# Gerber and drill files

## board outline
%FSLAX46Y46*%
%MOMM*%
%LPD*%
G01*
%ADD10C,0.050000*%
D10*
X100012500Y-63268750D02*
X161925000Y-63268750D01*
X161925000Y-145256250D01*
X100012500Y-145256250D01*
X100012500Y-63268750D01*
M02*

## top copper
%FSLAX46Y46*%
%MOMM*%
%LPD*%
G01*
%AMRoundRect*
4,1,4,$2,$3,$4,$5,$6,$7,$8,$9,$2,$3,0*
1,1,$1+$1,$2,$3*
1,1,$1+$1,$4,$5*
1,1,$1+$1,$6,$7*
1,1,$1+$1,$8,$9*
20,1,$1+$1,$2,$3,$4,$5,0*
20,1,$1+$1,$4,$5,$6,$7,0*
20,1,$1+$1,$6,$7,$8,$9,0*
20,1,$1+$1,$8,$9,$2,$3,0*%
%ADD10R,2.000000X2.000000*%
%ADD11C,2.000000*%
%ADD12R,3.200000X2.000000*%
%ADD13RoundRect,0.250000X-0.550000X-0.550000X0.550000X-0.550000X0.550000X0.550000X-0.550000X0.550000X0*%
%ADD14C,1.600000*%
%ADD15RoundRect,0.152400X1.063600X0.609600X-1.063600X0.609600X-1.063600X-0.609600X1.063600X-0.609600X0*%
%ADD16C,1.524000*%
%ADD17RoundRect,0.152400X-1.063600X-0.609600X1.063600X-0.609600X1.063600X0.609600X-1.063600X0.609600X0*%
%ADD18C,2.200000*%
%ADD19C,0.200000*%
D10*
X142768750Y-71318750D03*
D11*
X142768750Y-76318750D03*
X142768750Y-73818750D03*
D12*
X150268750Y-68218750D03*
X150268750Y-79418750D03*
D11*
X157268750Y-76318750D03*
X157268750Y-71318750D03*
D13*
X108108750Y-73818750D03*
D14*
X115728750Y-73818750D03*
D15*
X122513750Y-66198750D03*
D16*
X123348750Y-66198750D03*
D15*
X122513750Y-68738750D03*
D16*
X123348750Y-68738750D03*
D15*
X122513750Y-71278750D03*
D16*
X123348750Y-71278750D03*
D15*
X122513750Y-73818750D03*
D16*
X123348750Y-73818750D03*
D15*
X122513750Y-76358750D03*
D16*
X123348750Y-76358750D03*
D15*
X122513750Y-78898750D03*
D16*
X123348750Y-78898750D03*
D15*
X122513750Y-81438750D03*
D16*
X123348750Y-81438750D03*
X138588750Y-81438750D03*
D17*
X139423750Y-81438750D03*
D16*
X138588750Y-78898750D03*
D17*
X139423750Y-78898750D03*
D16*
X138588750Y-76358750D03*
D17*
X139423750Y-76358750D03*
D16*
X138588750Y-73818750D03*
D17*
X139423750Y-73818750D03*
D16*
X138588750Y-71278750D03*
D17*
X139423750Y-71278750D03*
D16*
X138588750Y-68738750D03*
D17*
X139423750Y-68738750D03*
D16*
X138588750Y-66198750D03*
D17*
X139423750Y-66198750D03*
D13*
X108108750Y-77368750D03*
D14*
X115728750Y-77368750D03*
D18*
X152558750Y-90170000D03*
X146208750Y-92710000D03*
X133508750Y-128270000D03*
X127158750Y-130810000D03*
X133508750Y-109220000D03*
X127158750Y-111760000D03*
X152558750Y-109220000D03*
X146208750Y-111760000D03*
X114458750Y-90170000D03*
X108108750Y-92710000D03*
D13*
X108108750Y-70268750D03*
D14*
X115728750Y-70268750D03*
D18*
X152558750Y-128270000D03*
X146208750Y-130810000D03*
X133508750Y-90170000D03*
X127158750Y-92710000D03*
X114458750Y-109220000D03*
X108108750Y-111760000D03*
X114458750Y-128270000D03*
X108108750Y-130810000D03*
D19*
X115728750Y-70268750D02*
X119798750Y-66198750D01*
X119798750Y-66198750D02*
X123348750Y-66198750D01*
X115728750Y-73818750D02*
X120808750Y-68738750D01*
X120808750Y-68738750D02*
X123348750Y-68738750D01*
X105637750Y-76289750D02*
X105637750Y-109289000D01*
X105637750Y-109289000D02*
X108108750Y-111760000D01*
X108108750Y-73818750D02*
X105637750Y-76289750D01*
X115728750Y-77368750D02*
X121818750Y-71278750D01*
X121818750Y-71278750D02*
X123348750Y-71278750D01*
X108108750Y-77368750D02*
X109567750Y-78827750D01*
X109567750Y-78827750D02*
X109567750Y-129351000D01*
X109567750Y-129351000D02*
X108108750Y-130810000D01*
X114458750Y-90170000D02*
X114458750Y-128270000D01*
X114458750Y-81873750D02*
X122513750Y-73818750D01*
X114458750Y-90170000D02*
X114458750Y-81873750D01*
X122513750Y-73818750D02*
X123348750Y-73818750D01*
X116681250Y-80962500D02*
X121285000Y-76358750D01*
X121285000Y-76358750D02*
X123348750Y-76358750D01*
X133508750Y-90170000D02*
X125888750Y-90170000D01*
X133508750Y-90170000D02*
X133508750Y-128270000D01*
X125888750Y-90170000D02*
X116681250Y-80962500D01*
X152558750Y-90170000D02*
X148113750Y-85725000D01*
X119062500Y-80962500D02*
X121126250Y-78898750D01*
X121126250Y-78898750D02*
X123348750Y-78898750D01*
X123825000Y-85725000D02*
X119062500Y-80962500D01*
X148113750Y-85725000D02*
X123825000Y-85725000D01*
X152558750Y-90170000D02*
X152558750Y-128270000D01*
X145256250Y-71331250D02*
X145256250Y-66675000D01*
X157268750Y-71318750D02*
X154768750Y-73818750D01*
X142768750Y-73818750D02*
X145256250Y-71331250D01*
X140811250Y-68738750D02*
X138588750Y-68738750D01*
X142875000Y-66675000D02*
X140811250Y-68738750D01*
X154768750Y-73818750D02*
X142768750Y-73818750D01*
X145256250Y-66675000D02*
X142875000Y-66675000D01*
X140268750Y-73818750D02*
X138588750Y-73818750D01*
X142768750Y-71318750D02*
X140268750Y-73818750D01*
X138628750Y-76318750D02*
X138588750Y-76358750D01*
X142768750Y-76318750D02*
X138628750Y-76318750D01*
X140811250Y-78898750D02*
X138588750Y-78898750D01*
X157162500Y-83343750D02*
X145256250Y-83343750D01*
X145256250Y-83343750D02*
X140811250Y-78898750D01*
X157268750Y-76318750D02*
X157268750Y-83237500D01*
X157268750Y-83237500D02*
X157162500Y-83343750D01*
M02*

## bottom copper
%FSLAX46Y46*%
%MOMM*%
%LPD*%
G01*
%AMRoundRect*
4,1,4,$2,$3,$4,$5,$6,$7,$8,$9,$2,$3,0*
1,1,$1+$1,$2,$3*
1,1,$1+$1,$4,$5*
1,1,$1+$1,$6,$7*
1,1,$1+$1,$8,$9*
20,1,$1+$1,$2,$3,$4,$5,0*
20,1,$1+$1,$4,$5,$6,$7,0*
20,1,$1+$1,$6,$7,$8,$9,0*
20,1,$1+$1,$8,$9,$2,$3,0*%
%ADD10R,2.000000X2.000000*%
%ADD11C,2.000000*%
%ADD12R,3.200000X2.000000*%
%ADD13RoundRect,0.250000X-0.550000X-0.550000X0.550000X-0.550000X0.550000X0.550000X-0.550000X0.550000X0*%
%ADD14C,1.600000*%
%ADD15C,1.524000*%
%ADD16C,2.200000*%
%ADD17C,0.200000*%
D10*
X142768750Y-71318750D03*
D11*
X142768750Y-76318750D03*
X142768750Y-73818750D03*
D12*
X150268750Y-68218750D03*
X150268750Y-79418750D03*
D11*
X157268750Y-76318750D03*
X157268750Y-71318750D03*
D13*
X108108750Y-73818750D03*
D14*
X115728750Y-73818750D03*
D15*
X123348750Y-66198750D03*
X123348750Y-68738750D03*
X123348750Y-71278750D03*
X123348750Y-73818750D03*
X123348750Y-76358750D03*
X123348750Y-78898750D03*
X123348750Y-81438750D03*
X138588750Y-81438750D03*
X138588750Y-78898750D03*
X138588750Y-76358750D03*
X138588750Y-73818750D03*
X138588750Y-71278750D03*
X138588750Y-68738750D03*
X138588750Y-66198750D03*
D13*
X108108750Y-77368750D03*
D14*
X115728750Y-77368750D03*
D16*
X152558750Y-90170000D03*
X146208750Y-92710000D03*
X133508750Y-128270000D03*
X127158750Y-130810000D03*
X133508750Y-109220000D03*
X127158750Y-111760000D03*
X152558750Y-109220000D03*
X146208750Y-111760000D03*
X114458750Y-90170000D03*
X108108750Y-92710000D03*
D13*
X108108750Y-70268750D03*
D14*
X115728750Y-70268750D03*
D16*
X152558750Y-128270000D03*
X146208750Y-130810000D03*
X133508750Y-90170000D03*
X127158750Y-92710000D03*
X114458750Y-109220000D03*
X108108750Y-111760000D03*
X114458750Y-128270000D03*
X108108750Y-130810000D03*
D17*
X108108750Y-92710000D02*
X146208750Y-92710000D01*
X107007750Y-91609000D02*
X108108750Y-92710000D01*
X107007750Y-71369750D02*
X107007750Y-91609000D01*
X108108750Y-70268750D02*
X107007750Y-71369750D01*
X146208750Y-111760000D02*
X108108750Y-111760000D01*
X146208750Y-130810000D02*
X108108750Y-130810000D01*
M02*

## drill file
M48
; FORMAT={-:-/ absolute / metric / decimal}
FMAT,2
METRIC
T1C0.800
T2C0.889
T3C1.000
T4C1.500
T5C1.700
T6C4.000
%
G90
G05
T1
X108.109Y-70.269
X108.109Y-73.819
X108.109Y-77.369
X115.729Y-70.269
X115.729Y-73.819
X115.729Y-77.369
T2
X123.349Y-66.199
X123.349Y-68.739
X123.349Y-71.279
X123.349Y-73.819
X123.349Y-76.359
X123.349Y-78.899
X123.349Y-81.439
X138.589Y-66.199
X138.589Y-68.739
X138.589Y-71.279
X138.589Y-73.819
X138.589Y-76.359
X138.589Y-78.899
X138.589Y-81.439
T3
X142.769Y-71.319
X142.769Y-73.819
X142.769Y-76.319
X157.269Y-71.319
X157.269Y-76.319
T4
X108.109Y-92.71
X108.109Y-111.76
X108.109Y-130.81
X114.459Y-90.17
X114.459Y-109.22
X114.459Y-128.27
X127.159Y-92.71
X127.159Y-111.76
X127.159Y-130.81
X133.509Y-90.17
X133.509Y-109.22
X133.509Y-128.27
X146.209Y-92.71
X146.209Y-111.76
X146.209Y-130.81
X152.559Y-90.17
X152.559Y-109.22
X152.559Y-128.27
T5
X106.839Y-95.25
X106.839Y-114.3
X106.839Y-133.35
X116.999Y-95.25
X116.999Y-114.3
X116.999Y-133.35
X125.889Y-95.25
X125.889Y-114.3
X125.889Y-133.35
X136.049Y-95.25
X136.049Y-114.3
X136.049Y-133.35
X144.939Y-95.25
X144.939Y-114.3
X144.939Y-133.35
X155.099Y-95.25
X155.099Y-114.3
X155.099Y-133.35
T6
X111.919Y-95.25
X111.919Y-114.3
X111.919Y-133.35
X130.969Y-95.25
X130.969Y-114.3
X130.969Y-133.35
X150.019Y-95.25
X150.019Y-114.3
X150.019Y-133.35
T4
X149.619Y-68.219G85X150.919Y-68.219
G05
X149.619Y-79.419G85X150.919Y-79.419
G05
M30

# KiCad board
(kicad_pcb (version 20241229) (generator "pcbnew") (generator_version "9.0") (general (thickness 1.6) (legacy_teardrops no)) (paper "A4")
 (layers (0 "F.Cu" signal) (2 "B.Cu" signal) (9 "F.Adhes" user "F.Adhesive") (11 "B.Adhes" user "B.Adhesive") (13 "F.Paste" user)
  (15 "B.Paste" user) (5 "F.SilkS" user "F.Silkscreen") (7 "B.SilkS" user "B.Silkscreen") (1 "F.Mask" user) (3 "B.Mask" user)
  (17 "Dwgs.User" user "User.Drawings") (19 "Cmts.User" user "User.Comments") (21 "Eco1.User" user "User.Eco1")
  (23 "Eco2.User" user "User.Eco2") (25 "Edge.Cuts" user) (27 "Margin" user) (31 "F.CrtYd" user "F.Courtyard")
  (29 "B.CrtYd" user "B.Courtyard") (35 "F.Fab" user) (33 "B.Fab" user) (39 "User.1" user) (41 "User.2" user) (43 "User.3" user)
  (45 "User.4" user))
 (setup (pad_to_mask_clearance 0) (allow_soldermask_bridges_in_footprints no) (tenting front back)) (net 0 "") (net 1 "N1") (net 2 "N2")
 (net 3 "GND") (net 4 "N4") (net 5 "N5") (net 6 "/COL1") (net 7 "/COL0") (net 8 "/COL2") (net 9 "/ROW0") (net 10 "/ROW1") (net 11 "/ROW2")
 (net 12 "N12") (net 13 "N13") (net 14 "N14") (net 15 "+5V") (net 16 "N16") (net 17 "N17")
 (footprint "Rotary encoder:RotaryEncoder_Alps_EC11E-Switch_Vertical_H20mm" (layer "F.Cu") (at 142.76875 71.31875)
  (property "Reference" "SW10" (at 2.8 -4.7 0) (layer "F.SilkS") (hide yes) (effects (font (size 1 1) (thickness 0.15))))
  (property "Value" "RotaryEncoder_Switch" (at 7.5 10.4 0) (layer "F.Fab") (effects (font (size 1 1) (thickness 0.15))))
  (pad "A" thru_hole rect (at 0 0) (size 2 2) (drill 1) (layers "*.Cu" "*.Mask") (remove_unused_layers no) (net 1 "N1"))
  (pad "B" thru_hole circle (at 0 5) (size 2 2) (drill 1) (layers "*.Cu" "*.Mask") (remove_unused_layers no) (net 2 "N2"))
  (pad "C" thru_hole circle (at 0 2.5) (size 2 2) (drill 1) (layers "*.Cu" "*.Mask") (remove_unused_layers no) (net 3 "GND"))
  (pad "MP" thru_hole rect (at 7.5 -3.1) (size 3.2 2) (drill oval 2.8 1.5) (layers "*.Cu" "*.Mask") (remove_unused_layers no))
  (pad "MP" thru_hole rect (at 7.5 8.1) (size 3.2 2) (drill oval 2.8 1.5) (layers "*.Cu" "*.Mask") (remove_unused_layers no))
  (pad "S1" thru_hole circle (at 14.5 5) (size 2 2) (drill 1) (layers "*.Cu" "*.Mask") (remove_unused_layers no) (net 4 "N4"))
  (pad "S2" thru_hole circle (at 14.5 0) (size 2 2) (drill 1) (layers "*.Cu" "*.Mask") (remove_unused_layers no) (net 3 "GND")))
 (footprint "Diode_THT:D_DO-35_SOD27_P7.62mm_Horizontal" (layer "F.Cu") (at 108.10875 73.81875)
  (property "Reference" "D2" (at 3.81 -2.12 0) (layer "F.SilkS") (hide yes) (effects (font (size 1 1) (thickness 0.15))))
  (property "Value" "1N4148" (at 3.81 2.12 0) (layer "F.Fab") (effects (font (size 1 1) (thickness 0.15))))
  (pad "1" thru_hole roundrect (at 0 0) (size 1.6 1.6) (drill 0.8) (layers "*.Cu" "*.Mask") (remove_unused_layers no)
   (roundrect_rratio 0.15625) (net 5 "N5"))
  (pad "2" thru_hole circle (at 7.62 0) (size 1.6 1.6) (drill 0.8) (layers "*.Cu" "*.Mask") (remove_unused_layers no) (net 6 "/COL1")))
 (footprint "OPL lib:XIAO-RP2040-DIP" (layer "F.Cu") (at 130.96875 73.81875)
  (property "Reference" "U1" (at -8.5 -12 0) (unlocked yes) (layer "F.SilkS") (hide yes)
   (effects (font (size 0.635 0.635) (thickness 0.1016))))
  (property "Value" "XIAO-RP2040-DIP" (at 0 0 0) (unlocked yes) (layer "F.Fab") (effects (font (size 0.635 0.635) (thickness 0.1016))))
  (pad "1" smd roundrect (at -8.455 -7.62 180) (size 2.432 1.524) (layers "F.Cu" "F.Mask") (roundrect_rratio 0.1) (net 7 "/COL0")
   (thermal_bridge_angle 45))
  (pad "1" thru_hole circle (at -7.62 -7.62 180) (size 1.524 1.524) (drill 0.889) (layers "*.Cu" "*.Mask") (remove_unused_layers no)
   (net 7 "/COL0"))
  (pad "2" smd roundrect (at -8.455 -5.08 180) (size 2.432 1.524) (layers "F.Cu" "F.Mask") (roundrect_rratio 0.1) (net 6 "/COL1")
   (thermal_bridge_angle 45))
  (pad "2" thru_hole circle (at -7.62 -5.08 180) (size 1.524 1.524) (drill 0.889) (layers "*.Cu" "*.Mask") (remove_unused_layers no)
   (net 6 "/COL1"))
  (pad "3" smd roundrect (at -8.455 -2.54 180) (size 2.432 1.524) (layers "F.Cu" "F.Mask") (roundrect_rratio 0.1) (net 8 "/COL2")
   (thermal_bridge_angle 45))
  (pad "3" thru_hole circle (at -7.62 -2.54 180) (size 1.524 1.524) (drill 0.889) (layers "*.Cu" "*.Mask") (remove_unused_layers no)
   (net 8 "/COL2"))
  (pad "4" smd roundrect (at -8.455 0 180) (size 2.432 1.524) (layers "F.Cu" "F.Mask") (roundrect_rratio 0.1) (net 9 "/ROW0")
   (thermal_bridge_angle 45))
  (pad "4" thru_hole circle (at -7.62 0 180) (size 1.524 1.524) (drill 0.889) (layers "*.Cu" "*.Mask") (remove_unused_layers no)
   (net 9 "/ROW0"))
  (pad "5" smd roundrect (at -8.455 2.54 180) (size 2.432 1.524) (layers "F.Cu" "F.Mask") (roundrect_rratio 0.1) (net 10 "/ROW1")
   (thermal_bridge_angle 45))
  (pad "5" thru_hole circle (at -7.62 2.54 180) (size 1.524 1.524) (drill 0.889) (layers "*.Cu" "*.Mask") (remove_unused_layers no)
   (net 10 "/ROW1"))
  (pad "6" smd roundrect (at -8.455 5.08 180) (size 2.432 1.524) (layers "F.Cu" "F.Mask") (roundrect_rratio 0.1) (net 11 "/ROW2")
   (thermal_bridge_angle 45))
  (pad "6" thru_hole circle (at -7.62 5.08 180) (size 1.524 1.524) (drill 0.889) (layers "*.Cu" "*.Mask") (remove_unused_layers no)
   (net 11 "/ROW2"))
  (pad "7" smd roundrect (at -8.455 7.62 180) (size 2.432 1.524) (layers "F.Cu" "F.Mask") (roundrect_rratio 0.1) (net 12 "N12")
   (thermal_bridge_angle 45))
  (pad "7" thru_hole circle (at -7.62 7.62 180) (size 1.524 1.524) (drill 0.889) (layers "*.Cu" "*.Mask") (remove_unused_layers no)
   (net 12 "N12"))
  (pad "8" thru_hole circle (at 7.62 7.62) (size 1.524 1.524) (drill 0.889) (layers "*.Cu" "*.Mask") (remove_unused_layers no)
   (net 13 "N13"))
  (pad "8" smd roundrect (at 8.455 7.62) (size 2.432 1.524) (layers "F.Cu" "F.Mask") (roundrect_rratio 0.1) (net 13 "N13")
   (thermal_bridge_angle 45))
  (pad "9" thru_hole circle (at 7.62 5.08) (size 1.524 1.524) (drill 0.889) (layers "*.Cu" "*.Mask") (remove_unused_layers no) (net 4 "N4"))
  (pad "9" smd roundrect (at 8.455 5.08) (size 2.432 1.524) (layers "F.Cu" "F.Mask") (roundrect_rratio 0.1) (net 4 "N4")
   (thermal_bridge_angle 45))
  (pad "10" thru_hole circle (at 7.62 2.54) (size 1.524 1.524) (drill 0.889) (layers "*.Cu" "*.Mask") (remove_unused_layers no) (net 2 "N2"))
  (pad "10" smd roundrect (at 8.455 2.54) (size 2.432 1.524) (layers "F.Cu" "F.Mask") (roundrect_rratio 0.1) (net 2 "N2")
   (thermal_bridge_angle 45))
  (pad "11" thru_hole circle (at 7.62 0) (size 1.524 1.524) (drill 0.889) (layers "*.Cu" "*.Mask") (remove_unused_layers no) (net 1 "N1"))
  (pad "11" smd roundrect (at 8.455 0) (size 2.432 1.524) (layers "F.Cu" "F.Mask") (roundrect_rratio 0.1) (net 1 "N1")
   (thermal_bridge_angle 45))
  (pad "12" thru_hole circle (at 7.62 -2.54) (size 1.524 1.524) (drill 0.889) (layers "*.Cu" "*.Mask") (remove_unused_layers no)
   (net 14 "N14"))
  (pad "12" smd roundrect (at 8.455 -2.54) (size 2.432 1.524) (layers "F.Cu" "F.Mask") (roundrect_rratio 0.1) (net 14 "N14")
   (thermal_bridge_angle 45))
  (pad "13" thru_hole circle (at 7.62 -5.08) (size 1.524 1.524) (drill 0.889) (layers "*.Cu" "*.Mask") (remove_unused_layers no)
   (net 3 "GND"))
  (pad "13" smd roundrect (at 8.455 -5.08) (size 2.432 1.524) (layers "F.Cu" "F.Mask") (roundrect_rratio 0.1) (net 3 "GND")
   (thermal_bridge_angle 45))
  (pad "14" thru_hole circle (at 7.62 -7.62) (size 1.524 1.524) (drill 0.889) (layers "*.Cu" "*.Mask") (remove_unused_layers no)
   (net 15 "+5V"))
  (pad "14" smd roundrect (at 8.455 -7.62) (size 2.432 1.524) (layers "F.Cu" "F.Mask") (roundrect_rratio 0.1) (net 15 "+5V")
   (thermal_bridge_angle 45)))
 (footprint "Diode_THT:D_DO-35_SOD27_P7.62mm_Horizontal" (layer "F.Cu") (at 108.10875 77.36875)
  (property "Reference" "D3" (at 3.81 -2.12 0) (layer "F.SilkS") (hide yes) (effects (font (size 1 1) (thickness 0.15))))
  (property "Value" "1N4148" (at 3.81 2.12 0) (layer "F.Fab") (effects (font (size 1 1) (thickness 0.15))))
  (pad "1" thru_hole roundrect (at 0 0) (size 1.6 1.6) (drill 0.8) (layers "*.Cu" "*.Mask") (remove_unused_layers no)
   (roundrect_rratio 0.15625) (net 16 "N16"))
  (pad "2" thru_hole circle (at 7.62 0) (size 1.6 1.6) (drill 0.8) (layers "*.Cu" "*.Mask") (remove_unused_layers no) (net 8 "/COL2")))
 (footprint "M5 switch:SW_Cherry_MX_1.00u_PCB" (layer "F.Cu") (at 152.55875 90.17)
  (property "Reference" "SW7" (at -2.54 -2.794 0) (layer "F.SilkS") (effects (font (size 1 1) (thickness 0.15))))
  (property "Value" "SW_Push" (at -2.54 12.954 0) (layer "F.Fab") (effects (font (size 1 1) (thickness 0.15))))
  (pad "" np_thru_hole circle (at -7.62 5.08) (size 1.7 1.7) (drill 1.7) (layers "*.Cu" "*.Mask"))
  (pad "" np_thru_hole circle (at -2.54 5.08) (size 4 4) (drill 4) (layers "*.Cu" "*.Mask"))
  (pad "" np_thru_hole circle (at 2.54 5.08) (size 1.7 1.7) (drill 1.7) (layers "*.Cu" "*.Mask"))
  (pad "1" thru_hole circle (at 0 0) (size 2.2 2.2) (drill 1.5) (layers "*.Cu" "*.Mask") (remove_unused_layers no) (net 11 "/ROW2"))
  (pad "2" thru_hole circle (at -6.35 2.54) (size 2.2 2.2) (drill 1.5) (layers "*.Cu" "*.Mask") (remove_unused_layers no) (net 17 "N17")))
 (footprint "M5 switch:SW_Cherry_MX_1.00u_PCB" (layer "F.Cu") (at 133.50875 128.27)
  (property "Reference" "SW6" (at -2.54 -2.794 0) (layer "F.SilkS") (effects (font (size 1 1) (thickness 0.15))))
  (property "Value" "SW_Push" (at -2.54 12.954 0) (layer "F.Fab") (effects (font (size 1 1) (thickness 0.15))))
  (pad "" np_thru_hole circle (at -7.62 5.08) (size 1.7 1.7) (drill 1.7) (layers "*.Cu" "*.Mask"))
  (pad "" np_thru_hole circle (at -2.54 5.08) (size 4 4) (drill 4) (layers "*.Cu" "*.Mask"))
  (pad "" np_thru_hole circle (at 2.54 5.08) (size 1.7 1.7) (drill 1.7) (layers "*.Cu" "*.Mask"))
  (pad "1" thru_hole circle (at 0 0) (size 2.2 2.2) (drill 1.5) (layers "*.Cu" "*.Mask") (remove_unused_layers no) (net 10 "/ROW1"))
  (pad "2" thru_hole circle (at -6.35 2.54) (size 2.2 2.2) (drill 1.5) (layers "*.Cu" "*.Mask") (remove_unused_layers no) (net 16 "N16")))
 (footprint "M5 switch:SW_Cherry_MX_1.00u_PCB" (layer "F.Cu") (at 133.50875 109.22)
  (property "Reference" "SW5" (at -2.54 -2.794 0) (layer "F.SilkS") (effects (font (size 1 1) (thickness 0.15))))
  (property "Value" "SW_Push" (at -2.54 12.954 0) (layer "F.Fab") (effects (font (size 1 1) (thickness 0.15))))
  (pad "" np_thru_hole circle (at -7.62 5.08) (size 1.7 1.7) (drill 1.7) (layers "*.Cu" "*.Mask"))
  (pad "" np_thru_hole circle (at -2.54 5.08) (size 4 4) (drill 4) (layers "*.Cu" "*.Mask"))
  (pad "" np_thru_hole circle (at 2.54 5.08) (size 1.7 1.7) (drill 1.7) (layers "*.Cu" "*.Mask"))
  (pad "1" thru_hole circle (at 0 0) (size 2.2 2.2) (drill 1.5) (layers "*.Cu" "*.Mask") (remove_unused_layers no) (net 10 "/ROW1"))
  (pad "2" thru_hole circle (at -6.35 2.54) (size 2.2 2.2) (drill 1.5) (layers "*.Cu" "*.Mask") (remove_unused_layers no) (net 5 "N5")))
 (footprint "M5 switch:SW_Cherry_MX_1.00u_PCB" (layer "F.Cu") (at 152.55875 109.22)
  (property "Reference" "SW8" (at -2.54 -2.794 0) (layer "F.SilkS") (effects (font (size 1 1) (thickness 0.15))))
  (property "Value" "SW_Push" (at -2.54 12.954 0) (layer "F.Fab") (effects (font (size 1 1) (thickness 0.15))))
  (pad "" np_thru_hole circle (at -7.62 5.08) (size 1.7 1.7) (drill 1.7) (layers "*.Cu" "*.Mask"))
  (pad "" np_thru_hole circle (at -2.54 5.08) (size 4 4) (drill 4) (layers "*.Cu" "*.Mask"))
  (pad "" np_thru_hole circle (at 2.54 5.08) (size 1.7 1.7) (drill 1.7) (layers "*.Cu" "*.Mask"))
  (pad "1" thru_hole circle (at 0 0) (size 2.2 2.2) (drill 1.5) (layers "*.Cu" "*.Mask") (remove_unused_layers no) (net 11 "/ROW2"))
  (pad "2" thru_hole circle (at -6.35 2.54) (size 2.2 2.2) (drill 1.5) (layers "*.Cu" "*.Mask") (remove_unused_layers no) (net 5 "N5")))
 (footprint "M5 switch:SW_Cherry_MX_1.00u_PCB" (layer "F.Cu") (at 114.45875 90.17)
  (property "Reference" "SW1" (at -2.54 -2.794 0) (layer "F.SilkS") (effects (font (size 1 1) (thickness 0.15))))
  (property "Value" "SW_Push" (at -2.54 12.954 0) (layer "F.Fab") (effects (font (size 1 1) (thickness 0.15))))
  (pad "" np_thru_hole circle (at -7.62 5.08) (size 1.7 1.7) (drill 1.7) (layers "*.Cu" "*.Mask"))
  (pad "" np_thru_hole circle (at -2.54 5.08) (size 4 4) (drill 4) (layers "*.Cu" "*.Mask"))
  (pad "" np_thru_hole circle (at 2.54 5.08) (size 1.7 1.7) (drill 1.7) (layers "*.Cu" "*.Mask"))
  (pad "1" thru_hole circle (at 0 0) (size 2.2 2.2) (drill 1.5) (layers "*.Cu" "*.Mask") (remove_unused_layers no) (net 9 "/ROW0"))
  (pad "2" thru_hole circle (at -6.35 2.54) (size 2.2 2.2) (drill 1.5) (layers "*.Cu" "*.Mask") (remove_unused_layers no) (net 17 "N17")))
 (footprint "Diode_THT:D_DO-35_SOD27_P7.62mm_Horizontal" (layer "F.Cu") (at 108.10875 70.26875)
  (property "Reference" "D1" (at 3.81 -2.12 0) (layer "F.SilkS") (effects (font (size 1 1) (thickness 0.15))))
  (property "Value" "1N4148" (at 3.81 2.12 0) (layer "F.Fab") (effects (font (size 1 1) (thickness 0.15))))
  (pad "1" thru_hole roundrect (at 0 0) (size 1.6 1.6) (drill 0.8) (layers "*.Cu" "*.Mask") (remove_unused_layers no)
   (roundrect_rratio 0.15625) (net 17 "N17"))
  (pad "2" thru_hole circle (at 7.62 0) (size 1.6 1.6) (drill 0.8) (layers "*.Cu" "*.Mask") (remove_unused_layers no) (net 7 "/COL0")))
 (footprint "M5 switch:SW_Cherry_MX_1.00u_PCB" (layer "F.Cu") (at 152.55875 128.27)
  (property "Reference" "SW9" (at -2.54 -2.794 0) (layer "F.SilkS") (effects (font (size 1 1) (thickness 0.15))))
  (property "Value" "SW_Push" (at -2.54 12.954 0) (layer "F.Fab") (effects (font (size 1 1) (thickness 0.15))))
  (pad "" np_thru_hole circle (at -7.62 5.08) (size 1.7 1.7) (drill 1.7) (layers "*.Cu" "*.Mask"))
  (pad "" np_thru_hole circle (at -2.54 5.08) (size 4 4) (drill 4) (layers "*.Cu" "*.Mask"))
  (pad "" np_thru_hole circle (at 2.54 5.08) (size 1.7 1.7) (drill 1.7) (layers "*.Cu" "*.Mask"))
  (pad "1" thru_hole circle (at 0 0) (size 2.2 2.2) (drill 1.5) (layers "*.Cu" "*.Mask") (remove_unused_layers no) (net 11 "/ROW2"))
  (pad "2" thru_hole circle (at -6.35 2.54) (size 2.2 2.2) (drill 1.5) (layers "*.Cu" "*.Mask") (remove_unused_layers no) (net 16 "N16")))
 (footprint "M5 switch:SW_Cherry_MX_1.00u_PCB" (layer "F.Cu") (at 133.50875 90.17)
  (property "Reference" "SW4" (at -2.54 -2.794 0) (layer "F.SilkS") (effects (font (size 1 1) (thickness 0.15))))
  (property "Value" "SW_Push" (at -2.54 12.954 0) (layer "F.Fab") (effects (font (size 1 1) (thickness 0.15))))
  (pad "" np_thru_hole circle (at -7.62 5.08) (size 1.7 1.7) (drill 1.7) (layers "*.Cu" "*.Mask"))
  (pad "" np_thru_hole circle (at -2.54 5.08) (size 4 4) (drill 4) (layers "*.Cu" "*.Mask"))
  (pad "" np_thru_hole circle (at 2.54 5.08) (size 1.7 1.7) (drill 1.7) (layers "*.Cu" "*.Mask"))
  (pad "1" thru_hole circle (at 0 0) (size 2.2 2.2) (drill 1.5) (layers "*.Cu" "*.Mask") (remove_unused_layers no) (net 10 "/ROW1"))
  (pad "2" thru_hole circle (at -6.35 2.54) (size 2.2 2.2) (drill 1.5) (layers "*.Cu" "*.Mask") (remove_unused_layers no) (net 17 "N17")))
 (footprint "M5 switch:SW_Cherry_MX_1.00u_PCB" (layer "F.Cu") (at 114.45875 109.22)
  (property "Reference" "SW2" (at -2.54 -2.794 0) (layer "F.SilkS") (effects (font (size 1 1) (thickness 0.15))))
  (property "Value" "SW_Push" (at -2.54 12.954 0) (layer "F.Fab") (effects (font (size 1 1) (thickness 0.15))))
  (pad "" np_thru_hole circle (at -7.62 5.08) (size 1.7 1.7) (drill 1.7) (layers "*.Cu" "*.Mask"))
  (pad "" np_thru_hole circle (at -2.54 5.08) (size 4 4) (drill 4) (layers "*.Cu" "*.Mask"))
  (pad "" np_thru_hole circle (at 2.54 5.08) (size 1.7 1.7) (drill 1.7) (layers "*.Cu" "*.Mask"))
  (pad "1" thru_hole circle (at 0 0) (size 2.2 2.2) (drill 1.5) (layers "*.Cu" "*.Mask") (remove_unused_layers no) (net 9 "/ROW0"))
  (pad "2" thru_hole circle (at -6.35 2.54) (size 2.2 2.2) (drill 1.5) (layers "*.Cu" "*.Mask") (remove_unused_layers no) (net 5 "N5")))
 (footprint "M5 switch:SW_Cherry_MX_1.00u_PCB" (layer "F.Cu") (at 114.45875 128.27)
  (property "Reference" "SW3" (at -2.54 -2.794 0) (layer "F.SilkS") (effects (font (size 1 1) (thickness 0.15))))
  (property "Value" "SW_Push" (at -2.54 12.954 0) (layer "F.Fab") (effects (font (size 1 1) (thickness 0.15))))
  (pad "" np_thru_hole circle (at -7.62 5.08) (size 1.7 1.7) (drill 1.7) (layers "*.Cu" "*.Mask"))
  (pad "" np_thru_hole circle (at -2.54 5.08) (size 4 4) (drill 4) (layers "*.Cu" "*.Mask"))
  (pad "" np_thru_hole circle (at 2.54 5.08) (size 1.7 1.7) (drill 1.7) (layers "*.Cu" "*.Mask"))
  (pad "1" thru_hole circle (at 0 0) (size 2.2 2.2) (drill 1.5) (layers "*.Cu" "*.Mask") (remove_unused_layers no) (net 9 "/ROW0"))
  (pad "2" thru_hole circle (at -6.35 2.54) (size 2.2 2.2) (drill 1.5) (layers "*.Cu" "*.Mask") (remove_unused_layers no) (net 16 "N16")))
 (gr_rect (start 100.0125 63.26875) (end 161.925 145.25625) (stroke (width 0.05) (type default)) (fill no) (layer "Edge.Cuts"))
 (segment (start 108.10875 92.71) (end 146.20875 92.71) (width 0.2) (layer "B.Cu") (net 17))
 (segment (start 107.00775 91.609) (end 108.10875 92.71) (width 0.2) (layer "B.Cu") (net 17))
 (segment (start 107.00775 71.36975) (end 107.00775 91.609) (width 0.2) (layer "B.Cu") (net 17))
 (segment (start 108.10875 70.26875) (end 107.00775 71.36975) (width 0.2) (layer "B.Cu") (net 17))
 (segment (start 115.72875 70.26875) (end 119.79875 66.19875) (width 0.2) (layer "F.Cu") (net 7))
 (segment (start 119.79875 66.19875) (end 123.34875 66.19875) (width 0.2) (layer "F.Cu") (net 7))
 (segment (start 115.72875 73.81875) (end 120.80875 68.73875) (width 0.2) (layer "F.Cu") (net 6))
 (segment (start 120.80875 68.73875) (end 123.34875 68.73875) (width 0.2) (layer "F.Cu") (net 6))
 (segment (start 105.63775 76.28975) (end 105.63775 109.289) (width 0.2) (layer "F.Cu") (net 5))
 (segment (start 105.63775 109.289) (end 108.10875 111.76) (width 0.2) (layer "F.Cu") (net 5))
 (segment (start 108.10875 73.81875) (end 105.63775 76.28975) (width 0.2) (layer "F.Cu") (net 5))
 (segment (start 146.20875 111.76) (end 108.10875 111.76) (width 0.2) (layer "B.Cu") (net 5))
 (segment (start 115.72875 77.36875) (end 121.81875 71.27875) (width 0.2) (layer "F.Cu") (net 8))
 (segment (start 121.81875 71.27875) (end 123.34875 71.27875) (width 0.2) (layer "F.Cu") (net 8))
 (segment (start 108.10875 77.36875) (end 109.56775 78.82775) (width 0.2) (layer "F.Cu") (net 16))
 (segment (start 109.56775 78.82775) (end 109.56775 129.351) (width 0.2) (layer "F.Cu") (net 16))
 (segment (start 109.56775 129.351) (end 108.10875 130.81) (width 0.2) (layer "F.Cu") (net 16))
 (segment (start 146.20875 130.81) (end 108.10875 130.81) (width 0.2) (layer "B.Cu") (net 16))
 (segment (start 114.45875 90.17) (end 114.45875 128.27) (width 0.2) (layer "F.Cu") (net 9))
 (segment (start 114.45875 81.87375) (end 122.51375 73.81875) (width 0.2) (layer "F.Cu") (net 9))
 (segment (start 114.45875 90.17) (end 114.45875 81.87375) (width 0.2) (layer "F.Cu") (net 9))
 (segment (start 122.51375 73.81875) (end 123.34875 73.81875) (width 0.2) (layer "F.Cu") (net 9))
 (segment (start 116.68125 80.9625) (end 121.285 76.35875) (width 0.2) (layer "F.Cu") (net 10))
 (segment (start 121.285 76.35875) (end 123.34875 76.35875) (width 0.2) (layer "F.Cu") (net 10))
 (segment (start 133.50875 90.17) (end 125.88875 90.17) (width 0.2) (layer "F.Cu") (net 10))
 (segment (start 133.50875 90.17) (end 133.50875 128.27) (width 0.2) (layer "F.Cu") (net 10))
 (segment (start 125.88875 90.17) (end 116.68125 80.9625) (width 0.2) (layer "F.Cu") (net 10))
 (segment (start 152.55875 90.17) (end 148.11375 85.725) (width 0.2) (layer "F.Cu") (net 11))
 (segment (start 119.0625 80.9625) (end 121.12625 78.89875) (width 0.2) (layer "F.Cu") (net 11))
 (segment (start 121.12625 78.89875) (end 123.34875 78.89875) (width 0.2) (layer "F.Cu") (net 11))
 (segment (start 123.825 85.725) (end 119.0625 80.9625) (width 0.2) (layer "F.Cu") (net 11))
 (segment (start 148.11375 85.725) (end 123.825 85.725) (width 0.2) (layer "F.Cu") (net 11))
 (segment (start 152.55875 90.17) (end 152.55875 128.27) (width 0.2) (layer "F.Cu") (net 11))
 (segment (start 145.25625 71.33125) (end 145.25625 66.675) (width 0.2) (layer "F.Cu") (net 3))
 (segment (start 157.26875 71.31875) (end 154.76875 73.81875) (width 0.2) (layer "F.Cu") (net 3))
 (segment (start 142.76875 73.81875) (end 145.25625 71.33125) (width 0.2) (layer "F.Cu") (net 3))
 (segment (start 140.81125 68.73875) (end 138.58875 68.73875) (width 0.2) (layer "F.Cu") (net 3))
 (segment (start 142.875 66.675) (end 140.81125 68.73875) (width 0.2) (layer "F.Cu") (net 3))
 (segment (start 154.76875 73.81875) (end 142.76875 73.81875) (width 0.2) (layer "F.Cu") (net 3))
 (segment (start 145.25625 66.675) (end 142.875 66.675) (width 0.2) (layer "F.Cu") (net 3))
 (segment (start 140.26875 73.81875) (end 138.58875 73.81875) (width 0.2) (layer "F.Cu") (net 1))
 (segment (start 142.76875 71.31875) (end 140.26875 73.81875) (width 0.2) (layer "F.Cu") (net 1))
 (segment (start 138.62875 76.31875) (end 138.58875 76.35875) (width 0.2) (layer "F.Cu") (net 2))
 (segment (start 142.76875 76.31875) (end 138.62875 76.31875) (width 0.2) (layer "F.Cu") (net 2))
 (segment (start 140.81125 78.89875) (end 138.58875 78.89875) (width 0.2) (layer "F.Cu") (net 4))
 (segment (start 157.1625 83.34375) (end 145.25625 83.34375) (width 0.2) (layer "F.Cu") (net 4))
 (segment (start 145.25625 83.34375) (end 140.81125 78.89875) (width 0.2) (layer "F.Cu") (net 4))
 (segment (start 157.26875 76.31875) (end 157.26875 83.2375) (width 0.2) (layer "F.Cu") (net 4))
 (segment (start 157.26875 83.2375) (end 157.1625 83.34375) (width 0.2) (layer "F.Cu") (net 4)))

